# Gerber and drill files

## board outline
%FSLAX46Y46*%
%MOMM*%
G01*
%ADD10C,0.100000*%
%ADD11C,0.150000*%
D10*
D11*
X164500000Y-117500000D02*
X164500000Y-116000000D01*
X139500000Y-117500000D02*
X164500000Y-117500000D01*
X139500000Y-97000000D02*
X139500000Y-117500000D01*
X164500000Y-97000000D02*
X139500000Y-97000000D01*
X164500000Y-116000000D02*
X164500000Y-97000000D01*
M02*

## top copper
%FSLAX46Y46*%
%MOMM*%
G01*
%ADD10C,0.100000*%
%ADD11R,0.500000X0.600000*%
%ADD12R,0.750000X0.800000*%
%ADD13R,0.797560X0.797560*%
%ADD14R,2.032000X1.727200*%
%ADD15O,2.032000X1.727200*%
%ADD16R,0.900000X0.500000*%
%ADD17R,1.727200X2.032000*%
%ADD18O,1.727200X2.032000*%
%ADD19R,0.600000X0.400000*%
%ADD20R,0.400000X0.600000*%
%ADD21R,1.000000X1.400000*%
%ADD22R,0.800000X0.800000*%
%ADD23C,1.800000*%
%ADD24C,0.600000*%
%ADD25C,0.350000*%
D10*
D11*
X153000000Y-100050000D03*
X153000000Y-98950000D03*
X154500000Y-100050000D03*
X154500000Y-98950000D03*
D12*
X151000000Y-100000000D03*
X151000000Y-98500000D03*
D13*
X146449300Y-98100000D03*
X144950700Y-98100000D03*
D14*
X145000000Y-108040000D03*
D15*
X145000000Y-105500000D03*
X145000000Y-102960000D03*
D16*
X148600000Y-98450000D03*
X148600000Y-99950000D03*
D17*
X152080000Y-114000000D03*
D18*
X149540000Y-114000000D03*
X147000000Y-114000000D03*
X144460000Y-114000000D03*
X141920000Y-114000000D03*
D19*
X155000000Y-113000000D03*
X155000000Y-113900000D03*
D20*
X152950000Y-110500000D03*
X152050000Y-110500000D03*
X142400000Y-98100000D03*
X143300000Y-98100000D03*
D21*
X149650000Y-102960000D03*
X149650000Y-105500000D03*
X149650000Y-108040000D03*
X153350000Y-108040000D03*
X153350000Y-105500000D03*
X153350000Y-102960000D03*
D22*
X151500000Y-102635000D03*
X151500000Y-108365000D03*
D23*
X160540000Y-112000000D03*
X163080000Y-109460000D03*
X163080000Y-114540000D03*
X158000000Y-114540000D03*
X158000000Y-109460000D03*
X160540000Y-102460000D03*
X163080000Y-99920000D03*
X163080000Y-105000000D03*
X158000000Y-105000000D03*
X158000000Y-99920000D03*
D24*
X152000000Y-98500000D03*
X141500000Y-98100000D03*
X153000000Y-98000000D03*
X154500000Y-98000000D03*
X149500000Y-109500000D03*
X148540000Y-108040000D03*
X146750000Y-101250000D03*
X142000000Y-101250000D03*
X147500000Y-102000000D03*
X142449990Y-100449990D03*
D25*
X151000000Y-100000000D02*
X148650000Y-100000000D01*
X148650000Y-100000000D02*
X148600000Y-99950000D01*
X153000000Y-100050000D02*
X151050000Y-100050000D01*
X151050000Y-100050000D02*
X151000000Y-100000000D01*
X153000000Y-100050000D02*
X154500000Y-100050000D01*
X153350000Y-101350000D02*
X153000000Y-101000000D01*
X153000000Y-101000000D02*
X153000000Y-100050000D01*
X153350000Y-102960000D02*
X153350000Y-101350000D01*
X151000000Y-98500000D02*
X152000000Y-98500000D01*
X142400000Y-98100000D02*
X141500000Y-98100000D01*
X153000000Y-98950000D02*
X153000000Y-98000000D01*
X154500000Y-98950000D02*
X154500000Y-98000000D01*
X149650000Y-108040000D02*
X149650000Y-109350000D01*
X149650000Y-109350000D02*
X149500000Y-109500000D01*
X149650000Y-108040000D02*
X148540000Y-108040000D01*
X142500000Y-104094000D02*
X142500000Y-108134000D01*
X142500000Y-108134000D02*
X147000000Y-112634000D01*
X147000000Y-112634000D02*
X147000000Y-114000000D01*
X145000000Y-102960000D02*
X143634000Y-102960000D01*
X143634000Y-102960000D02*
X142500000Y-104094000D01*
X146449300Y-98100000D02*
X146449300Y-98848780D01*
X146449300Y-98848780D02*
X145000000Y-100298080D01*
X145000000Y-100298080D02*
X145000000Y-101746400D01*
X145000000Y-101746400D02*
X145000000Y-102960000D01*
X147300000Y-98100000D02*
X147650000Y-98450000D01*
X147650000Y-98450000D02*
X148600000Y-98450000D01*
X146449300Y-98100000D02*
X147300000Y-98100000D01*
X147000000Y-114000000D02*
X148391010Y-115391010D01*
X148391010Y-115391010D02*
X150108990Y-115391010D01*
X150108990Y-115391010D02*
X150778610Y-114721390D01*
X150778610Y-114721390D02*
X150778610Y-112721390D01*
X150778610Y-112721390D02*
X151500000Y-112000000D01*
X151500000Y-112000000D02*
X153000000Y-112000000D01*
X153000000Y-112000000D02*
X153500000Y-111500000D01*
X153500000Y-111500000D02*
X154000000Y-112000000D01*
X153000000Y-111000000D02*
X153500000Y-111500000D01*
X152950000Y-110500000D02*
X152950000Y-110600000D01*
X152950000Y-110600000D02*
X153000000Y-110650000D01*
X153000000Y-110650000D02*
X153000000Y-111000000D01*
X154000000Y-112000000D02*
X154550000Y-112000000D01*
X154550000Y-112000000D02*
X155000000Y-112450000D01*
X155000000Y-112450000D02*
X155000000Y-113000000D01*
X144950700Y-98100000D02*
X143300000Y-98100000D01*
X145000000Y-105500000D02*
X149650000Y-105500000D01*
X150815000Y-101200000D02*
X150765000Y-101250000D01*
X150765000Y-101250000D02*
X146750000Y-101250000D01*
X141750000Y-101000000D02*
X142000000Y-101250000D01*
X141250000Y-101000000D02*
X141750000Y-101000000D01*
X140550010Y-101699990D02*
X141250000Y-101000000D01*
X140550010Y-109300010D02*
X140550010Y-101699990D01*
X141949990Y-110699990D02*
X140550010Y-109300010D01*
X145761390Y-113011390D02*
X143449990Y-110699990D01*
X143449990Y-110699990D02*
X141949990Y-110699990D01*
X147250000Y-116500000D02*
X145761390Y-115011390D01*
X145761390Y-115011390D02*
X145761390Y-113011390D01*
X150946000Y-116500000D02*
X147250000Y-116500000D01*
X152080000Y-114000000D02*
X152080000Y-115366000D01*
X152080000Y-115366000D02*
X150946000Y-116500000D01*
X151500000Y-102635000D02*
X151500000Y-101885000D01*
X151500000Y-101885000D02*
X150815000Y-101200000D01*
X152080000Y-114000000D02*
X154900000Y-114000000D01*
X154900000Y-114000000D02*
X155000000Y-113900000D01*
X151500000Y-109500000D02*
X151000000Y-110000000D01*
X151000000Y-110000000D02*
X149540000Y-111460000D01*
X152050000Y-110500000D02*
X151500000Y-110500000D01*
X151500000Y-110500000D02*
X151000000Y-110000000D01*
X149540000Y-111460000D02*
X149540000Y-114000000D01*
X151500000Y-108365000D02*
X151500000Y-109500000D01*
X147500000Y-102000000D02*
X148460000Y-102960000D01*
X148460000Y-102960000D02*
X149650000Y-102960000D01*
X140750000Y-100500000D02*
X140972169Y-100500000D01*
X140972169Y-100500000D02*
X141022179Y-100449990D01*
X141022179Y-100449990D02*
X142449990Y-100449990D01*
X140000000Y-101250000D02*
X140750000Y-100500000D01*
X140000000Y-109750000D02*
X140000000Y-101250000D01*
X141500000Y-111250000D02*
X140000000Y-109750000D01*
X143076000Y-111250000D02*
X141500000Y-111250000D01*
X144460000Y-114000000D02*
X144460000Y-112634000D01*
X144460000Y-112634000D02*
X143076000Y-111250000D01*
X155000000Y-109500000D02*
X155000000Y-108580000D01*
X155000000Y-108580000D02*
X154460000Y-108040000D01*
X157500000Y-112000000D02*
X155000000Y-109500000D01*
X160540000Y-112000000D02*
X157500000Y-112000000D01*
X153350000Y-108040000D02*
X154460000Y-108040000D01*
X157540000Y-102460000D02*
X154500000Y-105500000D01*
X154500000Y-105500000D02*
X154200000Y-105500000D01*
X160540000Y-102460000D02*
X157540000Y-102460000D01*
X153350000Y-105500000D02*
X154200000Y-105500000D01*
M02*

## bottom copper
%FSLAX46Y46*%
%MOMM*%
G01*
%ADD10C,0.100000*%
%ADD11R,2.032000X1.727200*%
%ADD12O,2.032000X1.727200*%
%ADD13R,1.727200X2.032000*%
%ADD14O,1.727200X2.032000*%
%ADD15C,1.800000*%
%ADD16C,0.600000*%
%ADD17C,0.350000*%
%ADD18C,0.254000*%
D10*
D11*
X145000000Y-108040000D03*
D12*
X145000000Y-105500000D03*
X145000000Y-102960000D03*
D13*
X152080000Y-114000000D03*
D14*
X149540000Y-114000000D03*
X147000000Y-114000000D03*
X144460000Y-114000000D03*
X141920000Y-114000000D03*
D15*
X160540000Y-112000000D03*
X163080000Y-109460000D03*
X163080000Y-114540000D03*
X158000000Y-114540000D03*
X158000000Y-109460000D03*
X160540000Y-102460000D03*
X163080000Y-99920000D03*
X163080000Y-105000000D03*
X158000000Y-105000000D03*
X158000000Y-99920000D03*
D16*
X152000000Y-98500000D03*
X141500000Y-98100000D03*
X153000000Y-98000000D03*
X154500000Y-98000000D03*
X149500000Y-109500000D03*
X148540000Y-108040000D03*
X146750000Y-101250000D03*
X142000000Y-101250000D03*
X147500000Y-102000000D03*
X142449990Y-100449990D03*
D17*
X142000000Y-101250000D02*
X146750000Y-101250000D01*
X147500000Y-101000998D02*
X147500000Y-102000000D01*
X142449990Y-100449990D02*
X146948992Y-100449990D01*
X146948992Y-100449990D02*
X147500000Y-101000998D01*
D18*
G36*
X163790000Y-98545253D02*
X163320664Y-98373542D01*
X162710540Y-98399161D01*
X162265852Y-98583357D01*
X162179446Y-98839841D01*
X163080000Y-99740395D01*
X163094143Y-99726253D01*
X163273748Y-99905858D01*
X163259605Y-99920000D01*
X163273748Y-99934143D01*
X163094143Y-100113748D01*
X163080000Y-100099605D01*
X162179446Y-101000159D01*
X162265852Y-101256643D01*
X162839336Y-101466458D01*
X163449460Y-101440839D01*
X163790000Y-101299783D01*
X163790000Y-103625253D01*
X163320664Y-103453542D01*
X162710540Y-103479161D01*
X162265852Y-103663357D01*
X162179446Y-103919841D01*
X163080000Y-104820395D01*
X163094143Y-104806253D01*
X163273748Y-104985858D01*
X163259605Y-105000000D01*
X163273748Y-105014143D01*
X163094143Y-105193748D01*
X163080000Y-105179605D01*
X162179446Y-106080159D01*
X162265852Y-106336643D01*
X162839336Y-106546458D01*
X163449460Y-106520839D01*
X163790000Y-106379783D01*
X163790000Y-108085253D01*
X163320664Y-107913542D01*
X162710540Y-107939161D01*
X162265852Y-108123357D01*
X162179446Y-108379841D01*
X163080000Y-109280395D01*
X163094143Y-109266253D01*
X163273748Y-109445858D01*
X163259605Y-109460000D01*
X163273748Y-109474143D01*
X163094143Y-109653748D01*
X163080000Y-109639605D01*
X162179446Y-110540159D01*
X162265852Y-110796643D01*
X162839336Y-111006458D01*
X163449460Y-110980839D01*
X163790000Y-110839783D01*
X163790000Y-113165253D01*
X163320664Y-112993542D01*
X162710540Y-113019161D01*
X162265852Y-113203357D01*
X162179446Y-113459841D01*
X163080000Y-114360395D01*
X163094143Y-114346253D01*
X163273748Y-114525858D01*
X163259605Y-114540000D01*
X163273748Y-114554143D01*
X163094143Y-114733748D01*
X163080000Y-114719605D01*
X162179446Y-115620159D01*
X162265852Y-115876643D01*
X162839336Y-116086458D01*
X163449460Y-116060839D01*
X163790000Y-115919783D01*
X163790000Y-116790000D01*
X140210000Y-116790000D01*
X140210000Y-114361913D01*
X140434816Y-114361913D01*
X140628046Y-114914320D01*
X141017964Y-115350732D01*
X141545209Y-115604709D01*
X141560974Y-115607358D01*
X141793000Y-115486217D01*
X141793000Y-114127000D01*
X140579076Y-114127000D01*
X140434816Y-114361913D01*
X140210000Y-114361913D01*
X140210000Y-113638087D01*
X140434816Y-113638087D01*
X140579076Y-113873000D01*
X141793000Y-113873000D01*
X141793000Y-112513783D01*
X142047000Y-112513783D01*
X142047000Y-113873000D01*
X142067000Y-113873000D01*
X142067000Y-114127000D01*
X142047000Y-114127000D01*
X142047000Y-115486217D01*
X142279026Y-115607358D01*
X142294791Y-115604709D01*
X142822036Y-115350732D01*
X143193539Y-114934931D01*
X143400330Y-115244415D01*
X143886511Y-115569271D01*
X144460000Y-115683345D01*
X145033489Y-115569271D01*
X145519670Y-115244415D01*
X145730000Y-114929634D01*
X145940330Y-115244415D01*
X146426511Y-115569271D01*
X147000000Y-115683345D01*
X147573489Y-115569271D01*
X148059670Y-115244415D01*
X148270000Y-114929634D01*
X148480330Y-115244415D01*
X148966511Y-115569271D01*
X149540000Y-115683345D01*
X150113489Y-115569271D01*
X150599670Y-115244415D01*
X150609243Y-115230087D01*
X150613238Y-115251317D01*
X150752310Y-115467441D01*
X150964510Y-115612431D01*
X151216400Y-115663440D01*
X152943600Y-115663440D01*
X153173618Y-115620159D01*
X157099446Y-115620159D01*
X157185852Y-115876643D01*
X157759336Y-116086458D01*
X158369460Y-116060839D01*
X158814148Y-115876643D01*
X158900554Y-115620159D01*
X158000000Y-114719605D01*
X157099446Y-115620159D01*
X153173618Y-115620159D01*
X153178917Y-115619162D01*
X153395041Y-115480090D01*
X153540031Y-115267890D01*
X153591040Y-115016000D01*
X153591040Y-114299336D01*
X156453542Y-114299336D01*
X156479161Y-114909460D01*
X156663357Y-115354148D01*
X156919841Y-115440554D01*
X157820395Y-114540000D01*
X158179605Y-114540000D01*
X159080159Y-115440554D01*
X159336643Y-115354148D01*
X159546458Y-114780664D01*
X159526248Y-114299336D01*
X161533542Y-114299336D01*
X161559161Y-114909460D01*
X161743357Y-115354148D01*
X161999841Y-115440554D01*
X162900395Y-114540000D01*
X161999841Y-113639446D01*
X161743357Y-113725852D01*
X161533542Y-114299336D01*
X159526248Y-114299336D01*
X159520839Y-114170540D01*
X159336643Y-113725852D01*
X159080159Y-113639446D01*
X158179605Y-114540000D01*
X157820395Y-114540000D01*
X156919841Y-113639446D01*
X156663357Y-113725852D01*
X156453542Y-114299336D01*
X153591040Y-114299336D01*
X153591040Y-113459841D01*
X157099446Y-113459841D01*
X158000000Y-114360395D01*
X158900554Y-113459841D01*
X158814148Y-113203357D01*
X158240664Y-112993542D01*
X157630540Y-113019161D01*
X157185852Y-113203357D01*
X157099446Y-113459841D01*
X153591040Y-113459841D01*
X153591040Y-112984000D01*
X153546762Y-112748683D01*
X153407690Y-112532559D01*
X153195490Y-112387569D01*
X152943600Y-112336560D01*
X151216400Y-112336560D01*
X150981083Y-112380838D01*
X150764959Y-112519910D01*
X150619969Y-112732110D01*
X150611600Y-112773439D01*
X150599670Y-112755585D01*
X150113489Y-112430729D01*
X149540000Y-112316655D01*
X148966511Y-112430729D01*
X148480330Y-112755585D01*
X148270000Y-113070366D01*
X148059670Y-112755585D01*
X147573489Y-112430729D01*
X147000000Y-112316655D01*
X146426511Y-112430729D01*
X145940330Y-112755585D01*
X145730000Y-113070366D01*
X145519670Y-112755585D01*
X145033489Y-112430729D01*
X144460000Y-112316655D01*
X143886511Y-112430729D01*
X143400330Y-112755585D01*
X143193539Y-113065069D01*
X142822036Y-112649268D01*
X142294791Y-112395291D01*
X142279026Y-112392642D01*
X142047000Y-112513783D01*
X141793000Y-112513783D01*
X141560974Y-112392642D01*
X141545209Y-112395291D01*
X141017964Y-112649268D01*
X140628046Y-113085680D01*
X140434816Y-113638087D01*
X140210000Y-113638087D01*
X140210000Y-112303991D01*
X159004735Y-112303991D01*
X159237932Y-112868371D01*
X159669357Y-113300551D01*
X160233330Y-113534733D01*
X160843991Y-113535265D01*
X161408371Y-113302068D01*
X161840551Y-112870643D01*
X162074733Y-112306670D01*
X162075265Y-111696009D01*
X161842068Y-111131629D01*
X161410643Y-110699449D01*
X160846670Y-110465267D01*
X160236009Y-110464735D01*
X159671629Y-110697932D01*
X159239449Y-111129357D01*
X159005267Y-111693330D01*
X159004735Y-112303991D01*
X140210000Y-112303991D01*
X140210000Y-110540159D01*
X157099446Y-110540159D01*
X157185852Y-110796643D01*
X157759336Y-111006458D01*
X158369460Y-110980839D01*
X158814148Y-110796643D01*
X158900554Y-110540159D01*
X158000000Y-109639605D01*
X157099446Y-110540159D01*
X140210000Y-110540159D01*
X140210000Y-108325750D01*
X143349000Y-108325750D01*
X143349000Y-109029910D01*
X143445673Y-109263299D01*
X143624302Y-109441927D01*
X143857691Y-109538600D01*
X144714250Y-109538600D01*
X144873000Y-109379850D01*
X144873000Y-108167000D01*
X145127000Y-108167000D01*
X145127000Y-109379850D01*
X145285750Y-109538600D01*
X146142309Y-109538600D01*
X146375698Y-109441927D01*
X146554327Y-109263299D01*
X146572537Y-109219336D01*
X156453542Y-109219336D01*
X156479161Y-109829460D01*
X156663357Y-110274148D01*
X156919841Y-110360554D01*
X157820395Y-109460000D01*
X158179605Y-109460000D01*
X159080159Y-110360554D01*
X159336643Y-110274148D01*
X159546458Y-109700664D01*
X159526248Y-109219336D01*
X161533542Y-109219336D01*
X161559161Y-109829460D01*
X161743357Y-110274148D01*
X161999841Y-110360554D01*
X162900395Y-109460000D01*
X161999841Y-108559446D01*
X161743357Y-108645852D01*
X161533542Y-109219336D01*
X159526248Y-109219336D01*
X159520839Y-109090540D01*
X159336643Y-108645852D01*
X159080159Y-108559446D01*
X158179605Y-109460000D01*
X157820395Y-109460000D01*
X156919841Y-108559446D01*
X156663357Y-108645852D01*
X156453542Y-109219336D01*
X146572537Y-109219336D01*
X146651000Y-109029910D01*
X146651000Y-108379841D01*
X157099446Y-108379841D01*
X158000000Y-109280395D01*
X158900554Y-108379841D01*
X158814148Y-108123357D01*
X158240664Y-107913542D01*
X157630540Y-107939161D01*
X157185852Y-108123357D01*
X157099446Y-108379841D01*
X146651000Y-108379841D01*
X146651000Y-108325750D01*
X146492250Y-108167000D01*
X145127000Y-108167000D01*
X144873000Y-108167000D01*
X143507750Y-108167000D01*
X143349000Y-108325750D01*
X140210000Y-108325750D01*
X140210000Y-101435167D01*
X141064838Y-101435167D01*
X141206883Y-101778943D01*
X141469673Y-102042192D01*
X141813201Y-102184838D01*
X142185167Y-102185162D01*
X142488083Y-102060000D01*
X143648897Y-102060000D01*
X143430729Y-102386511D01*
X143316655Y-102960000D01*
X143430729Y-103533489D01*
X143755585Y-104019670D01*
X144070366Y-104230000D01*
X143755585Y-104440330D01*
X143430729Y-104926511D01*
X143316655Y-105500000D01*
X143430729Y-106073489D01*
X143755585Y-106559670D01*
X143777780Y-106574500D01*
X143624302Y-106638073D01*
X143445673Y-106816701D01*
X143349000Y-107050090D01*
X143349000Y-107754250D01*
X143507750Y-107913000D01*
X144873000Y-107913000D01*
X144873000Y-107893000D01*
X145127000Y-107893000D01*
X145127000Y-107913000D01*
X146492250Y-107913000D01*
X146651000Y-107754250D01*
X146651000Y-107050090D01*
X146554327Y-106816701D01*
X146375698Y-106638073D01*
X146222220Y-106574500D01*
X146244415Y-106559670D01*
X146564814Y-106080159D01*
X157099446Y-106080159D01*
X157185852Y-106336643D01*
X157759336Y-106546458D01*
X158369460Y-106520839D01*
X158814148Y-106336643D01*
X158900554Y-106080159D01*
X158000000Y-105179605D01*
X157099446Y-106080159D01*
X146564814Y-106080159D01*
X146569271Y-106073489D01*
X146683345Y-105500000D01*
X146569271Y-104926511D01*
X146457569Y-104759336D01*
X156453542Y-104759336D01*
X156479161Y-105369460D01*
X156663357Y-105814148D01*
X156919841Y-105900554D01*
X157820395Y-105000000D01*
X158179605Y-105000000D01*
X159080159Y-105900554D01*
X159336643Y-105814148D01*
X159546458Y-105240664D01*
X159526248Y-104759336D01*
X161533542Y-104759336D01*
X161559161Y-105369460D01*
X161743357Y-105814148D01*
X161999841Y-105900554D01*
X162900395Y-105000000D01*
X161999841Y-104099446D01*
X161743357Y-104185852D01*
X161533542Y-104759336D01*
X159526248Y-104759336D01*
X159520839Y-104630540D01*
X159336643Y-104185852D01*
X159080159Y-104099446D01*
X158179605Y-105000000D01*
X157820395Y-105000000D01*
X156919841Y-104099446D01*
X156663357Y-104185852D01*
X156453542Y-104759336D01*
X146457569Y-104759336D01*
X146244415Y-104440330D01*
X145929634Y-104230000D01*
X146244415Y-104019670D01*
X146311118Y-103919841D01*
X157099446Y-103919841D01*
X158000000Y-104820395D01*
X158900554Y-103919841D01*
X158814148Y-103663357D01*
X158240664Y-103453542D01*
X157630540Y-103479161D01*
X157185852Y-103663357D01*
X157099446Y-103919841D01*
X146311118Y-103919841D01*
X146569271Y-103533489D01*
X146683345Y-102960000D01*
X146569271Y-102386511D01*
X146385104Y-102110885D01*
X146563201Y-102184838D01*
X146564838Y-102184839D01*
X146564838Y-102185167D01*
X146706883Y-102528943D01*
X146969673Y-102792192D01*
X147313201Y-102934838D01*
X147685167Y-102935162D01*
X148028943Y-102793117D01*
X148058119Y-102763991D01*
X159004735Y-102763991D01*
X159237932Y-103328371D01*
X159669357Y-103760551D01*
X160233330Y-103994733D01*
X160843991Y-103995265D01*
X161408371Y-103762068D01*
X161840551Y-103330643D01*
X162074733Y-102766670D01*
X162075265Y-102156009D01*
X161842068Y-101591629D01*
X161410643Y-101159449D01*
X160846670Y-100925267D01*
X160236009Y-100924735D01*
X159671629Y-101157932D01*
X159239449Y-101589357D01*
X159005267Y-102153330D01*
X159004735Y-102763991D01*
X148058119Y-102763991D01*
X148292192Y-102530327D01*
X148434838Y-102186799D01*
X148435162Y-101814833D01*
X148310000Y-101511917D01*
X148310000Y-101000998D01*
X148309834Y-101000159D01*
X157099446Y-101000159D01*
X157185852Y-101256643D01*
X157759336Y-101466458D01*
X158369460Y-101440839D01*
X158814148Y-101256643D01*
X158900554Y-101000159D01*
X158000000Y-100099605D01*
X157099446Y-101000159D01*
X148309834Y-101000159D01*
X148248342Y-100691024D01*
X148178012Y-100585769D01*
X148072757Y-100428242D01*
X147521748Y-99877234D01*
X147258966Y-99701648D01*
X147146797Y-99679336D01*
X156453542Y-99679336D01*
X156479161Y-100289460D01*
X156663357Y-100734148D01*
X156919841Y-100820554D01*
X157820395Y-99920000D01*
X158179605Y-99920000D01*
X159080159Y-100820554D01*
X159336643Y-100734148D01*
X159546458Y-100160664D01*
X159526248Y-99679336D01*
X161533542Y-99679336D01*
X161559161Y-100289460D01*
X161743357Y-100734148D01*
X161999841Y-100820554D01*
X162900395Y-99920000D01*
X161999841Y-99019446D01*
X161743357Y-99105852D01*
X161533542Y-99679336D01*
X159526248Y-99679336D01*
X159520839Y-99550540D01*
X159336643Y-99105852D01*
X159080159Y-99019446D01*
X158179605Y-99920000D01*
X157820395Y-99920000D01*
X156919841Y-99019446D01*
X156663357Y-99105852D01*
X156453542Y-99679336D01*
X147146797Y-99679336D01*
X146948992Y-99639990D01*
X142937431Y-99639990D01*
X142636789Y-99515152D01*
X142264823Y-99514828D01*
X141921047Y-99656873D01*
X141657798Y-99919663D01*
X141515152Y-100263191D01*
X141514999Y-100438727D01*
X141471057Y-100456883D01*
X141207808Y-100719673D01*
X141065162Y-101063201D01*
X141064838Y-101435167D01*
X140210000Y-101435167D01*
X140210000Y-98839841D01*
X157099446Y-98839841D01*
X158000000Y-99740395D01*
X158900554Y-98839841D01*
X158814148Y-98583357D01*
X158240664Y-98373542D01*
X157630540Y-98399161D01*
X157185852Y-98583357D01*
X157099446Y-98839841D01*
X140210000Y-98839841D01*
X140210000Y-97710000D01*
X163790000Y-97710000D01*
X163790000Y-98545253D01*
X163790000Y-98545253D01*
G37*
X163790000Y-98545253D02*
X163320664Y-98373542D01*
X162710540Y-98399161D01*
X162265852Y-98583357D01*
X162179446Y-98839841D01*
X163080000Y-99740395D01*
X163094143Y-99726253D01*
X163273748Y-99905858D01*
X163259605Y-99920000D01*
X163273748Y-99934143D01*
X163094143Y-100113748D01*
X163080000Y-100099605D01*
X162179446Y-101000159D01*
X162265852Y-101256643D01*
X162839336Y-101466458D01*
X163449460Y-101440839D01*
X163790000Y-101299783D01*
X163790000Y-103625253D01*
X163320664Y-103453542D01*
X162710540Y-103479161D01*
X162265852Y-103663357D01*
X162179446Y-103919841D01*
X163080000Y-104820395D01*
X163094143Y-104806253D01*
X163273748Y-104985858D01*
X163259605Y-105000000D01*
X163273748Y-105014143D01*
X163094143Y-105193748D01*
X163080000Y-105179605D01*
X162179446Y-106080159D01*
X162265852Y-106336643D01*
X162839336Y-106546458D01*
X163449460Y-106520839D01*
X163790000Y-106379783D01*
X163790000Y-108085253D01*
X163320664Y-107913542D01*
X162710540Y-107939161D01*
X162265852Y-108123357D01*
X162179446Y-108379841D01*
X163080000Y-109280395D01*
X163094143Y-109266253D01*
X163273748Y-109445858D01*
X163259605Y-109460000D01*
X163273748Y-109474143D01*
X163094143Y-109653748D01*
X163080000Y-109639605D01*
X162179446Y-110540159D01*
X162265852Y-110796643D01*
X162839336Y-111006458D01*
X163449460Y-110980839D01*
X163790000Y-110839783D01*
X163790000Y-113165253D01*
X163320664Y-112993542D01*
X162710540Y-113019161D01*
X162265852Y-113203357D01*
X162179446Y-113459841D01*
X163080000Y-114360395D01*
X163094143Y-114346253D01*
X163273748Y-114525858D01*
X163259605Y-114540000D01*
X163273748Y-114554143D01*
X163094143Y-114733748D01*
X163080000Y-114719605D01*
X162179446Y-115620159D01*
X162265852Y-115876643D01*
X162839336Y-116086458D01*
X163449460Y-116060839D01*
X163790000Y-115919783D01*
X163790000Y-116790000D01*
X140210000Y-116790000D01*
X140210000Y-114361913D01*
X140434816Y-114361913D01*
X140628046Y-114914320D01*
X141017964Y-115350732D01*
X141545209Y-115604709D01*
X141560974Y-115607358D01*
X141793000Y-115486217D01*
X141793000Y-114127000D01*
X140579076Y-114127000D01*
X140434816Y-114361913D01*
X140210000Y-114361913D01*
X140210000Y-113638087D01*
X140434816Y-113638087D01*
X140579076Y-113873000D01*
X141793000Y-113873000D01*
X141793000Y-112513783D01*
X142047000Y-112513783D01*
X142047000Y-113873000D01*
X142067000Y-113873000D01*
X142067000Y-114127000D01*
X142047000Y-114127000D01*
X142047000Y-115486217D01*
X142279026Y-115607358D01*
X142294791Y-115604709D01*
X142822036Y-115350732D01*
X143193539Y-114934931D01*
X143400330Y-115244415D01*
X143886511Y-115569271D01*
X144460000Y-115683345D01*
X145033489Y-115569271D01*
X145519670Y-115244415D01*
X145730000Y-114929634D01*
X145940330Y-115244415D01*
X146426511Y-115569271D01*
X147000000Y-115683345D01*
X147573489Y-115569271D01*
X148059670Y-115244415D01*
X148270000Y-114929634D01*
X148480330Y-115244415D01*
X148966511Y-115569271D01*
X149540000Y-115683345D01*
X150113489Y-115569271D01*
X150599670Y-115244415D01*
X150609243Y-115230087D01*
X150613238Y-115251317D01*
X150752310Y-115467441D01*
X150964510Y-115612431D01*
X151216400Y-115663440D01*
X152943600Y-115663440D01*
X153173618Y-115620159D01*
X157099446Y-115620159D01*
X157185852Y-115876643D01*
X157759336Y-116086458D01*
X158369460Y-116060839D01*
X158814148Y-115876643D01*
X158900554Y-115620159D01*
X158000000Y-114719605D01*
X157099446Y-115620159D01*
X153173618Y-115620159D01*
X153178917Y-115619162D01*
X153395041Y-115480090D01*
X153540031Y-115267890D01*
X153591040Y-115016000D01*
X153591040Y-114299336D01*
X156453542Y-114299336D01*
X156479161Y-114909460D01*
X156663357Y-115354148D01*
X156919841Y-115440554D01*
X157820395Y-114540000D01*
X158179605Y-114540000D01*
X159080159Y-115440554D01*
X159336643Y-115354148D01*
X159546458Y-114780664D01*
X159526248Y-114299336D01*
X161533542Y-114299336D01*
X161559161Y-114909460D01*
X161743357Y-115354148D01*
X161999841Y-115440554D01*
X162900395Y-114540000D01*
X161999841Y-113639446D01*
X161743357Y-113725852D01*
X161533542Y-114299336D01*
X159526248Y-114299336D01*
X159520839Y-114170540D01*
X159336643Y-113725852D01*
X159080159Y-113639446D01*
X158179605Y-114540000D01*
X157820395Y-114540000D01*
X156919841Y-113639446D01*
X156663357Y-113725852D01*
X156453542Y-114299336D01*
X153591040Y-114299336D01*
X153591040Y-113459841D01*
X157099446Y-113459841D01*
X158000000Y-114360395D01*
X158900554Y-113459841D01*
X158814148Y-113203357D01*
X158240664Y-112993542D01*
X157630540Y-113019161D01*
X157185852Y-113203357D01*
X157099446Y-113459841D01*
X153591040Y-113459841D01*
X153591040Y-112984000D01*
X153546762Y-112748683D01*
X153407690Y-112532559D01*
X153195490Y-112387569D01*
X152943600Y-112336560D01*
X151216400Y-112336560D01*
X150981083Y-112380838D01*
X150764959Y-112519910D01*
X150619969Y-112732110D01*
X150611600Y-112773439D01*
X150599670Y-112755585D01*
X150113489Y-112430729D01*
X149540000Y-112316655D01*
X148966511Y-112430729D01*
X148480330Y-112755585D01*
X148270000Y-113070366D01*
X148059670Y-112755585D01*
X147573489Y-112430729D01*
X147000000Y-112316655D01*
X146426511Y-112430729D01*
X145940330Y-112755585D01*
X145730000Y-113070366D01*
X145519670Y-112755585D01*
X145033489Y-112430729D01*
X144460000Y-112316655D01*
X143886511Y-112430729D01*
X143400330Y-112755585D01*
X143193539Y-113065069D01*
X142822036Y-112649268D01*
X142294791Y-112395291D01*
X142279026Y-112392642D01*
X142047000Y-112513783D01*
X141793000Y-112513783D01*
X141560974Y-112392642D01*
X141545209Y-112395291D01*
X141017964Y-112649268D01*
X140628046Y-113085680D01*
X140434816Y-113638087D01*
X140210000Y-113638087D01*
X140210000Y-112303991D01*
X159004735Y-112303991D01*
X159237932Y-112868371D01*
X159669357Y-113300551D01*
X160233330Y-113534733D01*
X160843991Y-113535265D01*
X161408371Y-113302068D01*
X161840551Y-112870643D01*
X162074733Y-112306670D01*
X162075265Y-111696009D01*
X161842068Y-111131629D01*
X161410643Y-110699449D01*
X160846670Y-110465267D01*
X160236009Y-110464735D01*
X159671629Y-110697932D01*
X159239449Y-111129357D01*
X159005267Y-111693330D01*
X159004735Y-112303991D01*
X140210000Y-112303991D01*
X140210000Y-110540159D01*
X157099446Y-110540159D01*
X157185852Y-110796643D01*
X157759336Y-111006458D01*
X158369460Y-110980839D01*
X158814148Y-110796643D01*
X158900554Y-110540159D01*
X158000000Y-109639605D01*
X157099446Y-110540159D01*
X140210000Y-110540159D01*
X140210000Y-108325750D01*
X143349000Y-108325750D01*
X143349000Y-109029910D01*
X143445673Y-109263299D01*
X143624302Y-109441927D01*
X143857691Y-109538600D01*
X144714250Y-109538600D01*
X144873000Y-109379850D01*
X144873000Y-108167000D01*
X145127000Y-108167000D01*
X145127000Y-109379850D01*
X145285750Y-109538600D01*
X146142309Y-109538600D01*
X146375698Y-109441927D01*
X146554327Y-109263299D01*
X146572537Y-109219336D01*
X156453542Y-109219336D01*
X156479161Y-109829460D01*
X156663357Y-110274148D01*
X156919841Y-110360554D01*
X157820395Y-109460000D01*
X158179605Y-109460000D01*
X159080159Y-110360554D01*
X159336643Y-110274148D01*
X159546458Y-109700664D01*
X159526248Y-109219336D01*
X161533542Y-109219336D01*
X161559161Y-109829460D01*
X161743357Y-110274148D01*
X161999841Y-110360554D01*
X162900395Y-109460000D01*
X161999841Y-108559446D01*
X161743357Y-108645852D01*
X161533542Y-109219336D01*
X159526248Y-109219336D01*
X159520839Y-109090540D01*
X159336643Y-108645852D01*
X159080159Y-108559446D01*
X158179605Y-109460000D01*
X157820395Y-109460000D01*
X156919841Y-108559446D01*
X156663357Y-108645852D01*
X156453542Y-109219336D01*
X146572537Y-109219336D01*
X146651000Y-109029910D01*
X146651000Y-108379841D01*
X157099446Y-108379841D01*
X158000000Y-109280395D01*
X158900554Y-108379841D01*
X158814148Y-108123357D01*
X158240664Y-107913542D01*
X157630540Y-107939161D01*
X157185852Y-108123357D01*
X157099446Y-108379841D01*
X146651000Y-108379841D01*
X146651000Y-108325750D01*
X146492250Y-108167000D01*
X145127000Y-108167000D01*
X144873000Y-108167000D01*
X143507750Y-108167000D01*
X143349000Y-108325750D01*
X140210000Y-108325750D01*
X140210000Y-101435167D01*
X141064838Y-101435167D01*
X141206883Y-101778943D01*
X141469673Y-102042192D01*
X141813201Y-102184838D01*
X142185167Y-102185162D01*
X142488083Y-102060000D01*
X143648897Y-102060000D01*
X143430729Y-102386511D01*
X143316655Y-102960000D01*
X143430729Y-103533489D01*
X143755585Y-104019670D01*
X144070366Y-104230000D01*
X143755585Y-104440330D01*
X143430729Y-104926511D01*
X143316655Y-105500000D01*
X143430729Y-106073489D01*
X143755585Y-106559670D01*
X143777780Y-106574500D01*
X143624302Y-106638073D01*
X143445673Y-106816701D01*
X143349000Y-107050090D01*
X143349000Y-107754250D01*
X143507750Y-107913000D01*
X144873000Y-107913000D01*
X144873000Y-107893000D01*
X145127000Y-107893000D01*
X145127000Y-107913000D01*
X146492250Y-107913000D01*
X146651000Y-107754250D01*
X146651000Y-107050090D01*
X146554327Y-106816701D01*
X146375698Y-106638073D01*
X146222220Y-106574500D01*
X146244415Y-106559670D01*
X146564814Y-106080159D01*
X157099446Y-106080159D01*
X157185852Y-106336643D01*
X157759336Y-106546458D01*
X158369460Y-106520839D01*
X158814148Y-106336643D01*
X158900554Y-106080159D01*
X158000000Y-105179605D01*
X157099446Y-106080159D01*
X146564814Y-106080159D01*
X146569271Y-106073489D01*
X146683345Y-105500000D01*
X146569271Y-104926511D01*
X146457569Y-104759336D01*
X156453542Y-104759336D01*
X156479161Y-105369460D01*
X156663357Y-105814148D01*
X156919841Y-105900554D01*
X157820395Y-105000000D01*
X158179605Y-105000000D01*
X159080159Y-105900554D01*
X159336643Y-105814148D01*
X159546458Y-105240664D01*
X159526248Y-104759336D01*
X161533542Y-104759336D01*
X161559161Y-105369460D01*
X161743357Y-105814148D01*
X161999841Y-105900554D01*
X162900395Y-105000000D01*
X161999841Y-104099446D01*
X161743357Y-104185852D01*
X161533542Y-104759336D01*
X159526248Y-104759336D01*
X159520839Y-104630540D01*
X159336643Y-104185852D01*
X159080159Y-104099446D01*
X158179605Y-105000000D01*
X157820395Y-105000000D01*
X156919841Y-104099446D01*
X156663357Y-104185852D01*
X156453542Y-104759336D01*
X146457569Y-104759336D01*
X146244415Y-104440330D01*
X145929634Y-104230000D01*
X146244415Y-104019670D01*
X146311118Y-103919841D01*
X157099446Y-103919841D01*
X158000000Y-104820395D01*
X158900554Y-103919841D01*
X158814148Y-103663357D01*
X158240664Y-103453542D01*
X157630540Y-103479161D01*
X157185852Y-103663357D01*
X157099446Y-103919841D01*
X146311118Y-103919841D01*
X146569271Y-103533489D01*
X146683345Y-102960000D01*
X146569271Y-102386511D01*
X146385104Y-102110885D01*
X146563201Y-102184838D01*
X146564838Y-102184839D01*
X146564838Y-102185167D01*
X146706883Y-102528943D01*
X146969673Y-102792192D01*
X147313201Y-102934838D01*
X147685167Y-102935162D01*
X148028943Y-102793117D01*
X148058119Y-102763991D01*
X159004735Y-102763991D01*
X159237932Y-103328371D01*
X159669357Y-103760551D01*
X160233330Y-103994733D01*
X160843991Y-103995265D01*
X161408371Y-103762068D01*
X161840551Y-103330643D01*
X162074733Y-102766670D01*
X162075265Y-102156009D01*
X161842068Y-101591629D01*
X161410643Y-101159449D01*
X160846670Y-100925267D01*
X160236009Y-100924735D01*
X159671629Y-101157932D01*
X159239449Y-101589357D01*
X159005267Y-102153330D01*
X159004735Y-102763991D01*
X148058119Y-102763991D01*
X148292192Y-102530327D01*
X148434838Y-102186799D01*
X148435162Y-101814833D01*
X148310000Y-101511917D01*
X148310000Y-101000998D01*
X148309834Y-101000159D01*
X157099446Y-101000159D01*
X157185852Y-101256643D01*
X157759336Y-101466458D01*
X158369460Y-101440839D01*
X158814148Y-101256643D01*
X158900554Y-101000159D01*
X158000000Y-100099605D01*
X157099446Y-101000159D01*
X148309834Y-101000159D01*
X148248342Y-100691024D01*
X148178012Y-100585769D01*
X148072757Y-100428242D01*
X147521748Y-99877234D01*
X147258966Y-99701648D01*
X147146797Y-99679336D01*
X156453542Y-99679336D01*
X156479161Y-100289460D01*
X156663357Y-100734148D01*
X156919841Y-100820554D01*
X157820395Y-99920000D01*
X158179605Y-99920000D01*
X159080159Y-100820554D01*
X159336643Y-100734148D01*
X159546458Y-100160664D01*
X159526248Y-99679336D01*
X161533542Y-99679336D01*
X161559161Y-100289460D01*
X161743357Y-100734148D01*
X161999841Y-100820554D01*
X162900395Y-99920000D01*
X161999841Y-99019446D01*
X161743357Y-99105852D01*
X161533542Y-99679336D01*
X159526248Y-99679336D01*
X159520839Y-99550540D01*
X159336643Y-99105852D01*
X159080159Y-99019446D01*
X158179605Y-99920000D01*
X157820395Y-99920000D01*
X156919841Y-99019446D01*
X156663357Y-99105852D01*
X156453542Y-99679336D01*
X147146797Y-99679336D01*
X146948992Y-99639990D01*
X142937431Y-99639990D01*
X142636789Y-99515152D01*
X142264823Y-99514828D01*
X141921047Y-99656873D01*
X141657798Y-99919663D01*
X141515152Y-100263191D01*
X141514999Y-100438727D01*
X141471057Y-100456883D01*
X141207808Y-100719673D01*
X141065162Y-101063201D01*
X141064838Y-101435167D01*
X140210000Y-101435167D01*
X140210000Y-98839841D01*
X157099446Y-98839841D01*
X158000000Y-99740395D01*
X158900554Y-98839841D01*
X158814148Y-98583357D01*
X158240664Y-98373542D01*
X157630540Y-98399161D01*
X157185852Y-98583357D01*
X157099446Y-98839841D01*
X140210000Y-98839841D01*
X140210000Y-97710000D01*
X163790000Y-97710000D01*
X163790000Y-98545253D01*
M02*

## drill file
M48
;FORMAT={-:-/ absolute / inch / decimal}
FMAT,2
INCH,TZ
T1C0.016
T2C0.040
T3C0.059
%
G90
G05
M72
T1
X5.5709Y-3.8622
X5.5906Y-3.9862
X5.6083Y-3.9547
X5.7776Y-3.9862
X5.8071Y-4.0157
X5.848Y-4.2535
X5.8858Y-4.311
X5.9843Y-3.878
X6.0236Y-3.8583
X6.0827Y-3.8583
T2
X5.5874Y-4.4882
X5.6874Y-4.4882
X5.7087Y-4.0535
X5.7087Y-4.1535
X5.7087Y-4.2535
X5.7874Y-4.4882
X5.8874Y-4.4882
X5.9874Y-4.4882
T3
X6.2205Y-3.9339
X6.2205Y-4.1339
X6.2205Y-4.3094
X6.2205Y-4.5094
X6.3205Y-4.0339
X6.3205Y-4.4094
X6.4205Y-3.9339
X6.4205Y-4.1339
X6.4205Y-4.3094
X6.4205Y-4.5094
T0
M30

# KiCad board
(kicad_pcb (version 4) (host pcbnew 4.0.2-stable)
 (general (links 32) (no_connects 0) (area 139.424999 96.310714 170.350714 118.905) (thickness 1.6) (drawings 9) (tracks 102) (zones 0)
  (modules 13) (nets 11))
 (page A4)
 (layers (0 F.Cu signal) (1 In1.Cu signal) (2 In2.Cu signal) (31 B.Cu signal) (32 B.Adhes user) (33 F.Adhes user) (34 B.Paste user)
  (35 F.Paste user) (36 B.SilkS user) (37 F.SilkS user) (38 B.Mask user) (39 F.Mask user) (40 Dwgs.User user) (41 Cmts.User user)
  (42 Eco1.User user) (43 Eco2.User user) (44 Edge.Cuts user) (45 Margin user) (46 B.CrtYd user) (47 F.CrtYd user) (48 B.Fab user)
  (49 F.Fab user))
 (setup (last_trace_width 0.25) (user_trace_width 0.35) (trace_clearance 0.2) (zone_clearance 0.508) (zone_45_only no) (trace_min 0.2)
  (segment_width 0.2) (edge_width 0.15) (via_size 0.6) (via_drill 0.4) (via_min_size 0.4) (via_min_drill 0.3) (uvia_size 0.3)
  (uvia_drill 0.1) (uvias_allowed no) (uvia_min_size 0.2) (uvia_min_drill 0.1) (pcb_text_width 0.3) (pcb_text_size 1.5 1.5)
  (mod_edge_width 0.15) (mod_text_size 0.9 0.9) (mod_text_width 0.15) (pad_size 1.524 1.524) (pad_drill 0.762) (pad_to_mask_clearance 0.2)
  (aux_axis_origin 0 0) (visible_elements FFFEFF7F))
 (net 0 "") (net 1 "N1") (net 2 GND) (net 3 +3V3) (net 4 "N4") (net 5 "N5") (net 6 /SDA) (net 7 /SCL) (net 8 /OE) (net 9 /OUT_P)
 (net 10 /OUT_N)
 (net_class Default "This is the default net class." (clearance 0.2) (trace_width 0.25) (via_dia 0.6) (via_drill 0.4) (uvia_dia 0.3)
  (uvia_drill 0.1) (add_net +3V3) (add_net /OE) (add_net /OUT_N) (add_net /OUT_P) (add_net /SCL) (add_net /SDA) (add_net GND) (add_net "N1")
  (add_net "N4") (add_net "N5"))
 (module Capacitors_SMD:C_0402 (layer F.Cu) (at 153 99.5 90)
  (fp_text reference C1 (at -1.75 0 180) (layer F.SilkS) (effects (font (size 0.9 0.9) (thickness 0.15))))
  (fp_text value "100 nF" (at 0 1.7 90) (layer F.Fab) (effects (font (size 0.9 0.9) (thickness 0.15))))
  (pad 1 smd rect (at -0.55 0 90) (size 0.6 0.5) (layers F.Cu F.Paste F.Mask) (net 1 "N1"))
  (pad 2 smd rect (at 0.55 0 90) (size 0.6 0.5) (layers F.Cu F.Paste F.Mask) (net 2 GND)))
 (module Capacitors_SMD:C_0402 (layer F.Cu) (at 154.5 99.5 90)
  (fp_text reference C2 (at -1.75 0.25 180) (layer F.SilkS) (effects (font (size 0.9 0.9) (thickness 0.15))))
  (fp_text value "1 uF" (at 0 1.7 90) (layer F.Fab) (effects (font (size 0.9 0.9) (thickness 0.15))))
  (pad 1 smd rect (at -0.55 0 90) (size 0.6 0.5) (layers F.Cu F.Paste F.Mask) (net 1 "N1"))
  (pad 2 smd rect (at 0.55 0 90) (size 0.6 0.5) (layers F.Cu F.Paste F.Mask) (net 2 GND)))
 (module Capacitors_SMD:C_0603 (layer F.Cu) (at 151 99.25 90)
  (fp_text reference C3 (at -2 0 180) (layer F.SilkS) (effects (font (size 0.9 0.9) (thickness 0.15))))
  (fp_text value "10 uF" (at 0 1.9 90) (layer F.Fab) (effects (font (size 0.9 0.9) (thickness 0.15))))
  (pad 1 smd rect (at -0.75 0 90) (size 0.8 0.75) (layers F.Cu F.Paste F.Mask) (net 1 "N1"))
  (pad 2 smd rect (at 0.75 0 90) (size 0.8 0.75) (layers F.Cu F.Paste F.Mask) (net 2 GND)))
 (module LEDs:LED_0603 (layer F.Cu) (at 145.7 98.1)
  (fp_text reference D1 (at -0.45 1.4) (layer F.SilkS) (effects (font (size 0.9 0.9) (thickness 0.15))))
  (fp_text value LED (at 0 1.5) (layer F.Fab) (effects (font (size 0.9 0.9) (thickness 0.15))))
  (pad 2 smd rect (at 0.7493 0 180) (size 0.79756 0.79756) (layers F.Cu F.Paste F.Mask) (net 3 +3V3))
  (pad 1 smd rect (at -0.7493 0 180) (size 0.79756 0.79756) (layers F.Cu F.Paste F.Mask) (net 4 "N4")))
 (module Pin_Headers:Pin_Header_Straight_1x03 (layer F.Cu) (at 145 108.04 180)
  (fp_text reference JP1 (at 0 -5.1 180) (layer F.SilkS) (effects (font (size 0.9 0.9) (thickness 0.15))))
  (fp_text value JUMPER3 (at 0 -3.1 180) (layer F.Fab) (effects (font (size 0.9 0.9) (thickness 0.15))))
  (pad 1 thru_hole rect (at 0 0 180) (size 2.032 1.7272) (drill 1.016) (layers *.Cu *.Mask F.SilkS) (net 2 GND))
  (pad 2 thru_hole oval (at 0 2.54 180) (size 2.032 1.7272) (drill 1.016) (layers *.Cu *.Mask F.SilkS) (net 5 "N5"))
  (pad 3 thru_hole oval (at 0 5.08 180) (size 2.032 1.7272) (drill 1.016) (layers *.Cu *.Mask F.SilkS) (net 3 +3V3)))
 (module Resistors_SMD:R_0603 (layer F.Cu) (at 148.6 99.2 270)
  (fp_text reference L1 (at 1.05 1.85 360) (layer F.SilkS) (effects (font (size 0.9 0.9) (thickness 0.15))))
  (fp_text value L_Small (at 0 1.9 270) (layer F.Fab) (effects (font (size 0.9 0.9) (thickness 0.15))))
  (pad 1 smd rect (at -0.75 0 270) (size 0.5 0.9) (layers F.Cu F.Paste F.Mask) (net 3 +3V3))
  (pad 2 smd rect (at 0.75 0 270) (size 0.5 0.9) (layers F.Cu F.Paste F.Mask) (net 1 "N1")))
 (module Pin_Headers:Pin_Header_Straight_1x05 (layer F.Cu) (at 152.08 114 270)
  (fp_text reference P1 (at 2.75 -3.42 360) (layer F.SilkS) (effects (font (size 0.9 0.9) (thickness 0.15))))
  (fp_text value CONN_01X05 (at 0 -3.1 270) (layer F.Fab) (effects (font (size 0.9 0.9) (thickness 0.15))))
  (pad 1 thru_hole rect (at 0 0 270) (size 2.032 1.7272) (drill 1.016) (layers *.Cu *.Mask F.SilkS) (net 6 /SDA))
  (pad 2 thru_hole oval (at 0 2.54 270) (size 2.032 1.7272) (drill 1.016) (layers *.Cu *.Mask F.SilkS) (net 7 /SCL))
  (pad 3 thru_hole oval (at 0 5.08 270) (size 2.032 1.7272) (drill 1.016) (layers *.Cu *.Mask F.SilkS) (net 3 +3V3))
  (pad 4 thru_hole oval (at 0 7.62 270) (size 2.032 1.7272) (drill 1.016) (layers *.Cu *.Mask F.SilkS) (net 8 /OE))
  (pad 5 thru_hole oval (at 0 10.16 270) (size 2.032 1.7272) (drill 1.016) (layers *.Cu *.Mask F.SilkS) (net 2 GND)))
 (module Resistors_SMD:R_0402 (layer F.Cu) (at 155 113.45 270)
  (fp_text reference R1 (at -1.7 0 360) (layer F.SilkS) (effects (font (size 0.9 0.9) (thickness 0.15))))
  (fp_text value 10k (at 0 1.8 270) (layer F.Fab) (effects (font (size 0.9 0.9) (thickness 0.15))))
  (pad 1 smd rect (at -0.45 0 270) (size 0.4 0.6) (layers F.Cu F.Paste F.Mask) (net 3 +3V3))
  (pad 2 smd rect (at 0.45 0 270) (size 0.4 0.6) (layers F.Cu F.Paste F.Mask) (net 6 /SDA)))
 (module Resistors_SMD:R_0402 (layer F.Cu) (at 152.5 110.5 180)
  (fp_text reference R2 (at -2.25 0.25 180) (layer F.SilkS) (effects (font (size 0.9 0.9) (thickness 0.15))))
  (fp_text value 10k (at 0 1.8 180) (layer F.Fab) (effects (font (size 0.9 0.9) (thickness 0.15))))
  (pad 1 smd rect (at -0.45 0 180) (size 0.4 0.6) (layers F.Cu F.Paste F.Mask) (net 3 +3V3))
  (pad 2 smd rect (at 0.45 0 180) (size 0.4 0.6) (layers F.Cu F.Paste F.Mask) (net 7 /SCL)))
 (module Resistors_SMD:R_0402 (layer F.Cu) (at 142.85 98.1)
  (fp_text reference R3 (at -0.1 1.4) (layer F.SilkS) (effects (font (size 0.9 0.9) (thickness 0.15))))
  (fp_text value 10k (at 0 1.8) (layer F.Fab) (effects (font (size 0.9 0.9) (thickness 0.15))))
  (pad 1 smd rect (at -0.45 0) (size 0.4 0.6) (layers F.Cu F.Paste F.Mask) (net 2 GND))
  (pad 2 smd rect (at 0.45 0) (size 0.4 0.6) (layers F.Cu F.Paste F.Mask) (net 4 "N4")))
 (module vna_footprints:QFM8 (layer F.Cu) (at 151.5 105.5)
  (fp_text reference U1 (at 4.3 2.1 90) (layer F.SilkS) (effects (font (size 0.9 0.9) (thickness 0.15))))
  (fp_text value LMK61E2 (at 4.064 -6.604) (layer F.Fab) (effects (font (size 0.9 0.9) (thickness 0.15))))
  (pad 1 smd rect (at -1.85 -2.54) (size 1 1.4) (layers F.Cu F.Paste F.Mask) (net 8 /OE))
  (pad 2 smd rect (at -1.85 0) (size 1 1.4) (layers F.Cu F.Paste F.Mask) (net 5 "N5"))
  (pad 3 smd rect (at -1.85 2.54) (size 1 1.4) (layers F.Cu F.Paste F.Mask) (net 2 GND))
  (pad 4 smd rect (at 1.85 2.54) (size 1 1.4) (layers F.Cu F.Paste F.Mask) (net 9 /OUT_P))
  (pad 5 smd rect (at 1.85 0) (size 1 1.4) (layers F.Cu F.Paste F.Mask) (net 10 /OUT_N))
  (pad 6 smd rect (at 1.85 -2.54) (size 1 1.4) (layers F.Cu F.Paste F.Mask) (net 1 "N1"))
  (pad 7 smd rect (at 0 -2.865) (size 0.8 0.8) (layers F.Cu F.Paste F.Mask) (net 6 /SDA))
  (pad 8 smd rect (at 0 2.865) (size 0.8 0.8) (layers F.Cu F.Paste F.Mask) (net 7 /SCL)))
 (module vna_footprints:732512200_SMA (layer F.Cu) (at 160.54 112 180)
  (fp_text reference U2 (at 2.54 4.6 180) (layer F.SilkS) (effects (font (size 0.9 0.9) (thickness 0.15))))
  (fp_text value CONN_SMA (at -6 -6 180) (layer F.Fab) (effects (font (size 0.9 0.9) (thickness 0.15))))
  (pad 1 thru_hole circle (at 0 0 180) (size 1.8 1.8) (drill 1.5) (layers *.Cu *.Mask F.SilkS) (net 9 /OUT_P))
  (pad 2 thru_hole circle (at -2.54 2.54 180) (size 1.8 1.8) (drill 1.5) (layers *.Cu *.Mask F.SilkS) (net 2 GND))
  (pad 3 thru_hole circle (at -2.54 -2.54 180) (size 1.8 1.8) (drill 1.5) (layers *.Cu *.Mask F.SilkS) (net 2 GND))
  (pad 4 thru_hole circle (at 2.54 -2.54 180) (size 1.8 1.8) (drill 1.5) (layers *.Cu *.Mask F.SilkS) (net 2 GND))
  (pad 5 thru_hole circle (at 2.54 2.54 180) (size 1.8 1.8) (drill 1.5) (layers *.Cu *.Mask F.SilkS) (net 2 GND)))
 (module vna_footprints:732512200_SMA (layer F.Cu) (at 160.54 102.46 180)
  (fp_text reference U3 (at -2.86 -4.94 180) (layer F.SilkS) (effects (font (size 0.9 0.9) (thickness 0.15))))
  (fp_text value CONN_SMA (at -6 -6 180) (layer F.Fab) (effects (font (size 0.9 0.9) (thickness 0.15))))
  (pad 1 thru_hole circle (at 0 0 180) (size 1.8 1.8) (drill 1.5) (layers *.Cu *.Mask F.SilkS) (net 10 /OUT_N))
  (pad 2 thru_hole circle (at -2.54 2.54 180) (size 1.8 1.8) (drill 1.5) (layers *.Cu *.Mask F.SilkS) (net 2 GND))
  (pad 3 thru_hole circle (at -2.54 -2.54 180) (size 1.8 1.8) (drill 1.5) (layers *.Cu *.Mask F.SilkS) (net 2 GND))
  (pad 4 thru_hole circle (at 2.54 -2.54 180) (size 1.8 1.8) (drill 1.5) (layers *.Cu *.Mask F.SilkS) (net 2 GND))
  (pad 5 thru_hole circle (at 2.54 2.54 180) (size 1.8 1.8) (drill 1.5) (layers *.Cu *.Mask F.SilkS) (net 2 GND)))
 (gr_line (start 164.5 117.5) (end 164.5 116) (layer Edge.Cuts) (width 0.15))
 (gr_line (start 139.5 117.5) (end 164.5 117.5) (layer Edge.Cuts) (width 0.15))
 (gr_line (start 139.5 97) (end 139.5 117.5) (layer Edge.Cuts) (width 0.15))
 (gr_line (start 164.5 97) (end 139.5 97) (layer Edge.Cuts) (width 0.15))
 (gr_line (start 164.5 116) (end 164.5 97) (layer Edge.Cuts) (width 0.15))
 (segment (start 151 100) (end 148.65 100) (width 0.35) (layer F.Cu) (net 1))
 (segment (start 148.65 100) (end 148.6 99.95) (width 0.35) (layer F.Cu) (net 1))
 (segment (start 153 100.05) (end 151.05 100.05) (width 0.35) (layer F.Cu) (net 1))
 (segment (start 151.05 100.05) (end 151 100) (width 0.35) (layer F.Cu) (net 1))
 (segment (start 153 100.05) (end 154.5 100.05) (width 0.35) (layer F.Cu) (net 1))
 (segment (start 153.35 101.35) (end 153 101) (width 0.35) (layer F.Cu) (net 1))
 (segment (start 153 101) (end 153 100.05) (width 0.35) (layer F.Cu) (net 1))
 (segment (start 153.35 102.96) (end 153.35 101.35) (width 0.35) (layer F.Cu) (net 1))
 (segment (start 151 98.5) (end 152 98.5) (width 0.35) (layer F.Cu) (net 2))
 (via (at 152 98.5) (size 0.6) (drill 0.4) (layers F.Cu B.Cu) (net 2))
 (via (at 141.5 98.1) (size 0.6) (drill 0.4) (layers F.Cu B.Cu) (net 2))
 (segment (start 142.4 98.1) (end 141.5 98.1) (width 0.35) (layer F.Cu) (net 2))
 (via (at 153 98) (size 0.6) (drill 0.4) (layers F.Cu B.Cu) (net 2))
 (segment (start 153 98.95) (end 153 98) (width 0.35) (layer F.Cu) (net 2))
 (segment (start 154.5 98.95) (end 154.5 98) (width 0.35) (layer F.Cu) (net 2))
 (via (at 154.5 98) (size 0.6) (drill 0.4) (layers F.Cu B.Cu) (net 2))
 (segment (start 149.65 108.04) (end 149.65 109.35) (width 0.35) (layer F.Cu) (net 2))
 (segment (start 149.65 109.35) (end 149.5 109.5) (width 0.35) (layer F.Cu) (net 2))
 (via (at 149.5 109.5) (size 0.6) (drill 0.4) (layers F.Cu B.Cu) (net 2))
 (via (at 148.54 108.04) (size 0.6) (drill 0.4) (layers F.Cu B.Cu) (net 2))
 (segment (start 149.65 108.04) (end 148.54 108.04) (width 0.35) (layer F.Cu) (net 2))
 (segment (start 142.5 104.094) (end 142.5 108.134) (width 0.35) (layer F.Cu) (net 3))
 (segment (start 142.5 108.134) (end 147 112.634) (width 0.35) (layer F.Cu) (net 3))
 (segment (start 147 112.634) (end 147 114) (width 0.35) (layer F.Cu) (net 3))
 (segment (start 145 102.96) (end 143.634 102.96) (width 0.35) (layer F.Cu) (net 3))
 (segment (start 143.634 102.96) (end 142.5 104.094) (width 0.35) (layer F.Cu) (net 3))
 (segment (start 146.4493 98.1) (end 146.4493 98.84878) (width 0.35) (layer F.Cu) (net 3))
 (segment (start 146.4493 98.84878) (end 145 100.29808) (width 0.35) (layer F.Cu) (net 3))
 (segment (start 145 100.29808) (end 145 101.7464) (width 0.35) (layer F.Cu) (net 3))
 (segment (start 145 101.7464) (end 145 102.96) (width 0.35) (layer F.Cu) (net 3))
 (segment (start 147.3 98.1) (end 147.65 98.45) (width 0.35) (layer F.Cu) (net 3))
 (segment (start 147.65 98.45) (end 148.6 98.45) (width 0.35) (layer F.Cu) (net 3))
 (segment (start 146.4493 98.1) (end 147.3 98.1) (width 0.35) (layer F.Cu) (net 3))
 (segment (start 147 114) (end 148.39101 115.39101) (width 0.35) (layer F.Cu) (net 3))
 (segment (start 148.39101 115.39101) (end 150.10899 115.39101) (width 0.35) (layer F.Cu) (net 3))
 (segment (start 150.10899 115.39101) (end 150.77861 114.72139) (width 0.35) (layer F.Cu) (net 3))
 (segment (start 150.77861 114.72139) (end 150.77861 112.72139) (width 0.35) (layer F.Cu) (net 3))
 (segment (start 150.77861 112.72139) (end 151.5 112) (width 0.35) (layer F.Cu) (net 3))
 (segment (start 151.5 112) (end 153 112) (width 0.35) (layer F.Cu) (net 3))
 (segment (start 153 112) (end 153.5 111.5) (width 0.35) (layer F.Cu) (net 3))
 (segment (start 153.5 111.5) (end 154 112) (width 0.35) (layer F.Cu) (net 3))
 (segment (start 153 111) (end 153.5 111.5) (width 0.35) (layer F.Cu) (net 3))
 (segment (start 152.95 110.5) (end 152.95 110.6) (width 0.35) (layer F.Cu) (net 3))
 (segment (start 152.95 110.6) (end 153 110.65) (width 0.35) (layer F.Cu) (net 3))
 (segment (start 153 110.65) (end 153 111) (width 0.35) (layer F.Cu) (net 3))
 (segment (start 154 112) (end 154.55 112) (width 0.35) (layer F.Cu) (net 3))
 (segment (start 154.55 112) (end 155 112.45) (width 0.35) (layer F.Cu) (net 3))
 (segment (start 155 112.45) (end 155 113) (width 0.35) (layer F.Cu) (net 3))
 (segment (start 144.9507 98.1) (end 143.3 98.1) (width 0.35) (layer F.Cu) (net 4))
 (segment (start 145 105.5) (end 149.65 105.5) (width 0.35) (layer F.Cu) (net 5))
 (segment (start 150.815 101.2) (end 150.765 101.25) (width 0.35) (layer F.Cu) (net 6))
 (segment (start 150.765 101.25) (end 146.75 101.25) (width 0.35) (layer F.Cu) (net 6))
 (via (at 146.75 101.25) (size 0.6) (drill 0.4) (layers F.Cu B.Cu) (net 6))
 (segment (start 142 101.25) (end 146.75 101.25) (width 0.35) (layer B.Cu) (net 6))
 (segment (start 141.75 101) (end 142 101.25) (width 0.35) (layer F.Cu) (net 6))
 (via (at 142 101.25) (size 0.6) (drill 0.4) (layers F.Cu B.Cu) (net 6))
 (segment (start 141.25 101) (end 141.75 101) (width 0.35) (layer F.Cu) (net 6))
 (segment (start 140.55001 101.69999) (end 141.25 101) (width 0.35) (layer F.Cu) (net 6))
 (segment (start 140.55001 109.30001) (end 140.55001 101.69999) (width 0.35) (layer F.Cu) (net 6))
 (segment (start 141.94999 110.69999) (end 140.55001 109.30001) (width 0.35) (layer F.Cu) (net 6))
 (segment (start 145.76139 113.01139) (end 143.44999 110.69999) (width 0.35) (layer F.Cu) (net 6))
 (segment (start 143.44999 110.69999) (end 141.94999 110.69999) (width 0.35) (layer F.Cu) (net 6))
 (segment (start 147.25 116.5) (end 145.76139 115.01139) (width 0.35) (layer F.Cu) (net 6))
 (segment (start 145.76139 115.01139) (end 145.76139 113.01139) (width 0.35) (layer F.Cu) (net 6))
 (segment (start 150.946 116.5) (end 147.25 116.5) (width 0.35) (layer F.Cu) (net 6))
 (segment (start 152.08 114) (end 152.08 115.366) (width 0.35) (layer F.Cu) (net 6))
 (segment (start 152.08 115.366) (end 150.946 116.5) (width 0.35) (layer F.Cu) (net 6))
 (segment (start 151.5 102.635) (end 151.5 101.885) (width 0.35) (layer F.Cu) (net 6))
 (segment (start 151.5 101.885) (end 150.815 101.2) (width 0.35) (layer F.Cu) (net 6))
 (segment (start 152.08 114) (end 154.9 114) (width 0.35) (layer F.Cu) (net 6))
 (segment (start 154.9 114) (end 155 113.9) (width 0.35) (layer F.Cu) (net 6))
 (segment (start 151.5 109.5) (end 151 110) (width 0.35) (layer F.Cu) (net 7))
 (segment (start 151 110) (end 149.54 111.46) (width 0.35) (layer F.Cu) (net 7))
 (segment (start 152.05 110.5) (end 151.5 110.5) (width 0.35) (layer F.Cu) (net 7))
 (segment (start 151.5 110.5) (end 151 110) (width 0.35) (layer F.Cu) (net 7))
 (segment (start 149.54 111.46) (end 149.54 114) (width 0.35) (layer F.Cu) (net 7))
 (segment (start 151.5 108.365) (end 151.5 109.5) (width 0.35) (layer F.Cu) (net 7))
 (segment (start 147.5 102) (end 148.46 102.96) (width 0.35) (layer F.Cu) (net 8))
 (segment (start 148.46 102.96) (end 149.65 102.96) (width 0.35) (layer F.Cu) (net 8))
 (segment (start 147.5 101.000998) (end 147.5 102) (width 0.35) (layer B.Cu) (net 8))
 (via (at 147.5 102) (size 0.6) (drill 0.4) (layers F.Cu B.Cu) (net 8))
 (segment (start 142.44999 100.44999) (end 146.948992 100.44999) (width 0.35) (layer B.Cu) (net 8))
 (segment (start 146.948992 100.44999) (end 147.5 101.000998) (width 0.35) (layer B.Cu) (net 8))
 (via (at 142.44999 100.44999) (size 0.6) (drill 0.4) (layers F.Cu B.Cu) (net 8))
 (segment (start 140.75 100.5) (end 140.972169 100.5) (width 0.35) (layer F.Cu) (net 8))
 (segment (start 140.972169 100.5) (end 141.022179 100.44999) (width 0.35) (layer F.Cu) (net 8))
 (segment (start 141.022179 100.44999) (end 142.44999 100.44999) (width 0.35) (layer F.Cu) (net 8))
 (segment (start 140 101.25) (end 140.75 100.5) (width 0.35) (layer F.Cu) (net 8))
 (segment (start 140 109.75) (end 140 101.25) (width 0.35) (layer F.Cu) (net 8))
 (segment (start 141.5 111.25) (end 140 109.75) (width 0.35) (layer F.Cu) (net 8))
 (segment (start 143.076 111.25) (end 141.5 111.25) (width 0.35) (layer F.Cu) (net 8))
 (segment (start 144.46 114) (end 144.46 112.634) (width 0.35) (layer F.Cu) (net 8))
 (segment (start 144.46 112.634) (end 143.076 111.25) (width 0.35) (layer F.Cu) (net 8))
 (segment (start 155 109.5) (end 155 108.58) (width 0.35) (layer F.Cu) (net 9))
 (segment (start 155 108.58) (end 154.46 108.04) (width 0.35) (layer F.Cu) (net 9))
 (segment (start 157.5 112) (end 155 109.5) (width 0.35) (layer F.Cu) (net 9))
 (segment (start 160.54 112) (end 157.5 112) (width 0.35) (layer F.Cu) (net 9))
 (segment (start 153.35 108.04) (end 154.46 108.04) (width 0.35) (layer F.Cu) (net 9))
 (segment (start 157.54 102.46) (end 154.5 105.5) (width 0.35) (layer F.Cu) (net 10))
 (segment (start 154.5 105.5) (end 154.2 105.5) (width 0.35) (layer F.Cu) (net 10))
 (segment (start 160.54 102.46) (end 157.54 102.46) (width 0.35) (layer F.Cu) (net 10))
 (segment (start 153.35 105.5) (end 154.2 105.5) (width 0.35) (layer F.Cu) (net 10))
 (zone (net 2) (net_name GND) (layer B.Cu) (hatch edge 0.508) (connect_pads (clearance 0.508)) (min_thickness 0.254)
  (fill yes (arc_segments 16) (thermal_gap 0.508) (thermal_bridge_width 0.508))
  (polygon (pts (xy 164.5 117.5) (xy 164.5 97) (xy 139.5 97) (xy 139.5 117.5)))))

